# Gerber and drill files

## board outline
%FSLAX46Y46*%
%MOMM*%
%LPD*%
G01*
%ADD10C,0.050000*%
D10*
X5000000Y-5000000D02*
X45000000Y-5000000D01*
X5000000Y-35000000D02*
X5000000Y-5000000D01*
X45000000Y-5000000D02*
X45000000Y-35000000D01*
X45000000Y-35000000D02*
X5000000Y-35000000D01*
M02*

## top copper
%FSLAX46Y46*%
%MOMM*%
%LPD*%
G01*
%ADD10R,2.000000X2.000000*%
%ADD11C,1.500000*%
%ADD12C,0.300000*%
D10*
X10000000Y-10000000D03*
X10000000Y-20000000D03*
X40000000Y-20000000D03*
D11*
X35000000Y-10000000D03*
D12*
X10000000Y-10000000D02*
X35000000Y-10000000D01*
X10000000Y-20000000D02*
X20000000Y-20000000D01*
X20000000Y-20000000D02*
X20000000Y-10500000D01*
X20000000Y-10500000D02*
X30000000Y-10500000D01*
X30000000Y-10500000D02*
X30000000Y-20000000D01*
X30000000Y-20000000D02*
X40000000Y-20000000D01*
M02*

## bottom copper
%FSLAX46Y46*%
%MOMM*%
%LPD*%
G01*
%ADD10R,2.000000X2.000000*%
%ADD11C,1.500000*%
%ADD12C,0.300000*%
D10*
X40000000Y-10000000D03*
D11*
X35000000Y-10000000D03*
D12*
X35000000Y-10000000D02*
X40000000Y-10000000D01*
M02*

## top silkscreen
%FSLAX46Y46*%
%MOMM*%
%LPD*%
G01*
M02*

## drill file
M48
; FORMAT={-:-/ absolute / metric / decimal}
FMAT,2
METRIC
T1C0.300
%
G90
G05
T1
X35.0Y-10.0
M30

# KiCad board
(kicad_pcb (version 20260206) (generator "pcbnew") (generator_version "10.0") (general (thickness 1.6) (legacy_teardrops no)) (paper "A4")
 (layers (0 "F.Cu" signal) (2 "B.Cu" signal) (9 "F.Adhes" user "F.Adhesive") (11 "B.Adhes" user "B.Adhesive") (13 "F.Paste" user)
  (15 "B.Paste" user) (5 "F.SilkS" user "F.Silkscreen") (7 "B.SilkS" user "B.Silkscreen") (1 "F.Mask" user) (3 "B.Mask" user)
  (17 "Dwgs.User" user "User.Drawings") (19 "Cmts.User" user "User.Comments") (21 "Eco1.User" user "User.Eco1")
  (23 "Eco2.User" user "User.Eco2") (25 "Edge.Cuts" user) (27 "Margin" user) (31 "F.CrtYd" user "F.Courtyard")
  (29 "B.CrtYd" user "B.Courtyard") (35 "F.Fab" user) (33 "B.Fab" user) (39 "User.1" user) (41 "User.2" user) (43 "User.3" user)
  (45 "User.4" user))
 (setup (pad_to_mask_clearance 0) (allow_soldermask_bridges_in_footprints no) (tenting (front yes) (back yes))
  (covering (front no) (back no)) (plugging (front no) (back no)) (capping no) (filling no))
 (gr_line (start 5 5) (end 45 5) (stroke (width 0.05) (type default)) (layer "Edge.Cuts"))
 (gr_line (start 5 35) (end 5 5) (stroke (width 0.05) (type default)) (layer "Edge.Cuts"))
 (gr_line (start 45 5) (end 45 35) (stroke (width 0.05) (type default)) (layer "Edge.Cuts"))
 (gr_line (start 45 35) (end 5 35) (stroke (width 0.05) (type default)) (layer "Edge.Cuts"))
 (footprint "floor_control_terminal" (layer "F.Cu") (at 10 10)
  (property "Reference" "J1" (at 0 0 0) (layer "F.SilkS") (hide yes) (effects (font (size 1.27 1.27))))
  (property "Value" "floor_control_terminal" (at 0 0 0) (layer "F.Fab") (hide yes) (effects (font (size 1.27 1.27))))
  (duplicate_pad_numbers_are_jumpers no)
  (pad "1" smd rect (at 0 0) (size 2 2) (layers "F.Cu" "F.Paste" "F.Mask") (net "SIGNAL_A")))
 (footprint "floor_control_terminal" (layer "B.Cu") (at 40 10)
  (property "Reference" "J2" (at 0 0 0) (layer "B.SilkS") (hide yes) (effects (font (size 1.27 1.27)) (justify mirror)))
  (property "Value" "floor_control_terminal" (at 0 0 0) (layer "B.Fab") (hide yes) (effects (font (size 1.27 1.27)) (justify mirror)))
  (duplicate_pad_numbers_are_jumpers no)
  (pad "1" smd rect (at 0 0) (size 2 2) (layers "B.Cu" "B.Paste" "B.Mask") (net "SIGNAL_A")))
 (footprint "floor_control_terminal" (layer "F.Cu") (at 10 20)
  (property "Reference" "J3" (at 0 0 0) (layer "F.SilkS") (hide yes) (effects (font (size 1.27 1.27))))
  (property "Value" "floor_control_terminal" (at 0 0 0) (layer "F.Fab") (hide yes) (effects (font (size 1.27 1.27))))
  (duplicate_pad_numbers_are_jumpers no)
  (pad "1" smd rect (at 0 0) (size 2 2) (layers "F.Cu" "F.Paste" "F.Mask") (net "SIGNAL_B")))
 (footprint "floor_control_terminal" (layer "F.Cu") (at 40 20)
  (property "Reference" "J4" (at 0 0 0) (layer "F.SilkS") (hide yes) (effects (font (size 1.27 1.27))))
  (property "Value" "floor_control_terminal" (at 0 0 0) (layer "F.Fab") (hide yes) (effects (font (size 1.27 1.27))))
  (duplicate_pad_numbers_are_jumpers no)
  (pad "1" smd rect (at 0 0) (size 2 2) (layers "F.Cu" "F.Paste" "F.Mask") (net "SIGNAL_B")))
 (segment (start 10 10) (end 35 10) (width 0.3) (layer "F.Cu") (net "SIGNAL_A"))
 (segment (start 35 10) (end 40 10) (width 0.3) (layer "B.Cu") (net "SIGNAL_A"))
 (via (at 35 10) (size 1.5) (drill 0.3) (layers "F.Cu" "B.Cu") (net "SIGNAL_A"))
 (segment (start 10 20) (end 20 20) (width 0.3) (layer "F.Cu") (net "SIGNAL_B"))
 (segment (start 20 20) (end 20 10.5) (width 0.3) (layer "F.Cu") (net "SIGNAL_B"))
 (segment (start 20 10.5) (end 30 10.5) (width 0.3) (layer "F.Cu") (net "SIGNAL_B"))
 (segment (start 30 10.5) (end 30 20) (width 0.3) (layer "F.Cu") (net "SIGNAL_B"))
 (segment (start 30 20) (end 40 20) (width 0.3) (layer "F.Cu") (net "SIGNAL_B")))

